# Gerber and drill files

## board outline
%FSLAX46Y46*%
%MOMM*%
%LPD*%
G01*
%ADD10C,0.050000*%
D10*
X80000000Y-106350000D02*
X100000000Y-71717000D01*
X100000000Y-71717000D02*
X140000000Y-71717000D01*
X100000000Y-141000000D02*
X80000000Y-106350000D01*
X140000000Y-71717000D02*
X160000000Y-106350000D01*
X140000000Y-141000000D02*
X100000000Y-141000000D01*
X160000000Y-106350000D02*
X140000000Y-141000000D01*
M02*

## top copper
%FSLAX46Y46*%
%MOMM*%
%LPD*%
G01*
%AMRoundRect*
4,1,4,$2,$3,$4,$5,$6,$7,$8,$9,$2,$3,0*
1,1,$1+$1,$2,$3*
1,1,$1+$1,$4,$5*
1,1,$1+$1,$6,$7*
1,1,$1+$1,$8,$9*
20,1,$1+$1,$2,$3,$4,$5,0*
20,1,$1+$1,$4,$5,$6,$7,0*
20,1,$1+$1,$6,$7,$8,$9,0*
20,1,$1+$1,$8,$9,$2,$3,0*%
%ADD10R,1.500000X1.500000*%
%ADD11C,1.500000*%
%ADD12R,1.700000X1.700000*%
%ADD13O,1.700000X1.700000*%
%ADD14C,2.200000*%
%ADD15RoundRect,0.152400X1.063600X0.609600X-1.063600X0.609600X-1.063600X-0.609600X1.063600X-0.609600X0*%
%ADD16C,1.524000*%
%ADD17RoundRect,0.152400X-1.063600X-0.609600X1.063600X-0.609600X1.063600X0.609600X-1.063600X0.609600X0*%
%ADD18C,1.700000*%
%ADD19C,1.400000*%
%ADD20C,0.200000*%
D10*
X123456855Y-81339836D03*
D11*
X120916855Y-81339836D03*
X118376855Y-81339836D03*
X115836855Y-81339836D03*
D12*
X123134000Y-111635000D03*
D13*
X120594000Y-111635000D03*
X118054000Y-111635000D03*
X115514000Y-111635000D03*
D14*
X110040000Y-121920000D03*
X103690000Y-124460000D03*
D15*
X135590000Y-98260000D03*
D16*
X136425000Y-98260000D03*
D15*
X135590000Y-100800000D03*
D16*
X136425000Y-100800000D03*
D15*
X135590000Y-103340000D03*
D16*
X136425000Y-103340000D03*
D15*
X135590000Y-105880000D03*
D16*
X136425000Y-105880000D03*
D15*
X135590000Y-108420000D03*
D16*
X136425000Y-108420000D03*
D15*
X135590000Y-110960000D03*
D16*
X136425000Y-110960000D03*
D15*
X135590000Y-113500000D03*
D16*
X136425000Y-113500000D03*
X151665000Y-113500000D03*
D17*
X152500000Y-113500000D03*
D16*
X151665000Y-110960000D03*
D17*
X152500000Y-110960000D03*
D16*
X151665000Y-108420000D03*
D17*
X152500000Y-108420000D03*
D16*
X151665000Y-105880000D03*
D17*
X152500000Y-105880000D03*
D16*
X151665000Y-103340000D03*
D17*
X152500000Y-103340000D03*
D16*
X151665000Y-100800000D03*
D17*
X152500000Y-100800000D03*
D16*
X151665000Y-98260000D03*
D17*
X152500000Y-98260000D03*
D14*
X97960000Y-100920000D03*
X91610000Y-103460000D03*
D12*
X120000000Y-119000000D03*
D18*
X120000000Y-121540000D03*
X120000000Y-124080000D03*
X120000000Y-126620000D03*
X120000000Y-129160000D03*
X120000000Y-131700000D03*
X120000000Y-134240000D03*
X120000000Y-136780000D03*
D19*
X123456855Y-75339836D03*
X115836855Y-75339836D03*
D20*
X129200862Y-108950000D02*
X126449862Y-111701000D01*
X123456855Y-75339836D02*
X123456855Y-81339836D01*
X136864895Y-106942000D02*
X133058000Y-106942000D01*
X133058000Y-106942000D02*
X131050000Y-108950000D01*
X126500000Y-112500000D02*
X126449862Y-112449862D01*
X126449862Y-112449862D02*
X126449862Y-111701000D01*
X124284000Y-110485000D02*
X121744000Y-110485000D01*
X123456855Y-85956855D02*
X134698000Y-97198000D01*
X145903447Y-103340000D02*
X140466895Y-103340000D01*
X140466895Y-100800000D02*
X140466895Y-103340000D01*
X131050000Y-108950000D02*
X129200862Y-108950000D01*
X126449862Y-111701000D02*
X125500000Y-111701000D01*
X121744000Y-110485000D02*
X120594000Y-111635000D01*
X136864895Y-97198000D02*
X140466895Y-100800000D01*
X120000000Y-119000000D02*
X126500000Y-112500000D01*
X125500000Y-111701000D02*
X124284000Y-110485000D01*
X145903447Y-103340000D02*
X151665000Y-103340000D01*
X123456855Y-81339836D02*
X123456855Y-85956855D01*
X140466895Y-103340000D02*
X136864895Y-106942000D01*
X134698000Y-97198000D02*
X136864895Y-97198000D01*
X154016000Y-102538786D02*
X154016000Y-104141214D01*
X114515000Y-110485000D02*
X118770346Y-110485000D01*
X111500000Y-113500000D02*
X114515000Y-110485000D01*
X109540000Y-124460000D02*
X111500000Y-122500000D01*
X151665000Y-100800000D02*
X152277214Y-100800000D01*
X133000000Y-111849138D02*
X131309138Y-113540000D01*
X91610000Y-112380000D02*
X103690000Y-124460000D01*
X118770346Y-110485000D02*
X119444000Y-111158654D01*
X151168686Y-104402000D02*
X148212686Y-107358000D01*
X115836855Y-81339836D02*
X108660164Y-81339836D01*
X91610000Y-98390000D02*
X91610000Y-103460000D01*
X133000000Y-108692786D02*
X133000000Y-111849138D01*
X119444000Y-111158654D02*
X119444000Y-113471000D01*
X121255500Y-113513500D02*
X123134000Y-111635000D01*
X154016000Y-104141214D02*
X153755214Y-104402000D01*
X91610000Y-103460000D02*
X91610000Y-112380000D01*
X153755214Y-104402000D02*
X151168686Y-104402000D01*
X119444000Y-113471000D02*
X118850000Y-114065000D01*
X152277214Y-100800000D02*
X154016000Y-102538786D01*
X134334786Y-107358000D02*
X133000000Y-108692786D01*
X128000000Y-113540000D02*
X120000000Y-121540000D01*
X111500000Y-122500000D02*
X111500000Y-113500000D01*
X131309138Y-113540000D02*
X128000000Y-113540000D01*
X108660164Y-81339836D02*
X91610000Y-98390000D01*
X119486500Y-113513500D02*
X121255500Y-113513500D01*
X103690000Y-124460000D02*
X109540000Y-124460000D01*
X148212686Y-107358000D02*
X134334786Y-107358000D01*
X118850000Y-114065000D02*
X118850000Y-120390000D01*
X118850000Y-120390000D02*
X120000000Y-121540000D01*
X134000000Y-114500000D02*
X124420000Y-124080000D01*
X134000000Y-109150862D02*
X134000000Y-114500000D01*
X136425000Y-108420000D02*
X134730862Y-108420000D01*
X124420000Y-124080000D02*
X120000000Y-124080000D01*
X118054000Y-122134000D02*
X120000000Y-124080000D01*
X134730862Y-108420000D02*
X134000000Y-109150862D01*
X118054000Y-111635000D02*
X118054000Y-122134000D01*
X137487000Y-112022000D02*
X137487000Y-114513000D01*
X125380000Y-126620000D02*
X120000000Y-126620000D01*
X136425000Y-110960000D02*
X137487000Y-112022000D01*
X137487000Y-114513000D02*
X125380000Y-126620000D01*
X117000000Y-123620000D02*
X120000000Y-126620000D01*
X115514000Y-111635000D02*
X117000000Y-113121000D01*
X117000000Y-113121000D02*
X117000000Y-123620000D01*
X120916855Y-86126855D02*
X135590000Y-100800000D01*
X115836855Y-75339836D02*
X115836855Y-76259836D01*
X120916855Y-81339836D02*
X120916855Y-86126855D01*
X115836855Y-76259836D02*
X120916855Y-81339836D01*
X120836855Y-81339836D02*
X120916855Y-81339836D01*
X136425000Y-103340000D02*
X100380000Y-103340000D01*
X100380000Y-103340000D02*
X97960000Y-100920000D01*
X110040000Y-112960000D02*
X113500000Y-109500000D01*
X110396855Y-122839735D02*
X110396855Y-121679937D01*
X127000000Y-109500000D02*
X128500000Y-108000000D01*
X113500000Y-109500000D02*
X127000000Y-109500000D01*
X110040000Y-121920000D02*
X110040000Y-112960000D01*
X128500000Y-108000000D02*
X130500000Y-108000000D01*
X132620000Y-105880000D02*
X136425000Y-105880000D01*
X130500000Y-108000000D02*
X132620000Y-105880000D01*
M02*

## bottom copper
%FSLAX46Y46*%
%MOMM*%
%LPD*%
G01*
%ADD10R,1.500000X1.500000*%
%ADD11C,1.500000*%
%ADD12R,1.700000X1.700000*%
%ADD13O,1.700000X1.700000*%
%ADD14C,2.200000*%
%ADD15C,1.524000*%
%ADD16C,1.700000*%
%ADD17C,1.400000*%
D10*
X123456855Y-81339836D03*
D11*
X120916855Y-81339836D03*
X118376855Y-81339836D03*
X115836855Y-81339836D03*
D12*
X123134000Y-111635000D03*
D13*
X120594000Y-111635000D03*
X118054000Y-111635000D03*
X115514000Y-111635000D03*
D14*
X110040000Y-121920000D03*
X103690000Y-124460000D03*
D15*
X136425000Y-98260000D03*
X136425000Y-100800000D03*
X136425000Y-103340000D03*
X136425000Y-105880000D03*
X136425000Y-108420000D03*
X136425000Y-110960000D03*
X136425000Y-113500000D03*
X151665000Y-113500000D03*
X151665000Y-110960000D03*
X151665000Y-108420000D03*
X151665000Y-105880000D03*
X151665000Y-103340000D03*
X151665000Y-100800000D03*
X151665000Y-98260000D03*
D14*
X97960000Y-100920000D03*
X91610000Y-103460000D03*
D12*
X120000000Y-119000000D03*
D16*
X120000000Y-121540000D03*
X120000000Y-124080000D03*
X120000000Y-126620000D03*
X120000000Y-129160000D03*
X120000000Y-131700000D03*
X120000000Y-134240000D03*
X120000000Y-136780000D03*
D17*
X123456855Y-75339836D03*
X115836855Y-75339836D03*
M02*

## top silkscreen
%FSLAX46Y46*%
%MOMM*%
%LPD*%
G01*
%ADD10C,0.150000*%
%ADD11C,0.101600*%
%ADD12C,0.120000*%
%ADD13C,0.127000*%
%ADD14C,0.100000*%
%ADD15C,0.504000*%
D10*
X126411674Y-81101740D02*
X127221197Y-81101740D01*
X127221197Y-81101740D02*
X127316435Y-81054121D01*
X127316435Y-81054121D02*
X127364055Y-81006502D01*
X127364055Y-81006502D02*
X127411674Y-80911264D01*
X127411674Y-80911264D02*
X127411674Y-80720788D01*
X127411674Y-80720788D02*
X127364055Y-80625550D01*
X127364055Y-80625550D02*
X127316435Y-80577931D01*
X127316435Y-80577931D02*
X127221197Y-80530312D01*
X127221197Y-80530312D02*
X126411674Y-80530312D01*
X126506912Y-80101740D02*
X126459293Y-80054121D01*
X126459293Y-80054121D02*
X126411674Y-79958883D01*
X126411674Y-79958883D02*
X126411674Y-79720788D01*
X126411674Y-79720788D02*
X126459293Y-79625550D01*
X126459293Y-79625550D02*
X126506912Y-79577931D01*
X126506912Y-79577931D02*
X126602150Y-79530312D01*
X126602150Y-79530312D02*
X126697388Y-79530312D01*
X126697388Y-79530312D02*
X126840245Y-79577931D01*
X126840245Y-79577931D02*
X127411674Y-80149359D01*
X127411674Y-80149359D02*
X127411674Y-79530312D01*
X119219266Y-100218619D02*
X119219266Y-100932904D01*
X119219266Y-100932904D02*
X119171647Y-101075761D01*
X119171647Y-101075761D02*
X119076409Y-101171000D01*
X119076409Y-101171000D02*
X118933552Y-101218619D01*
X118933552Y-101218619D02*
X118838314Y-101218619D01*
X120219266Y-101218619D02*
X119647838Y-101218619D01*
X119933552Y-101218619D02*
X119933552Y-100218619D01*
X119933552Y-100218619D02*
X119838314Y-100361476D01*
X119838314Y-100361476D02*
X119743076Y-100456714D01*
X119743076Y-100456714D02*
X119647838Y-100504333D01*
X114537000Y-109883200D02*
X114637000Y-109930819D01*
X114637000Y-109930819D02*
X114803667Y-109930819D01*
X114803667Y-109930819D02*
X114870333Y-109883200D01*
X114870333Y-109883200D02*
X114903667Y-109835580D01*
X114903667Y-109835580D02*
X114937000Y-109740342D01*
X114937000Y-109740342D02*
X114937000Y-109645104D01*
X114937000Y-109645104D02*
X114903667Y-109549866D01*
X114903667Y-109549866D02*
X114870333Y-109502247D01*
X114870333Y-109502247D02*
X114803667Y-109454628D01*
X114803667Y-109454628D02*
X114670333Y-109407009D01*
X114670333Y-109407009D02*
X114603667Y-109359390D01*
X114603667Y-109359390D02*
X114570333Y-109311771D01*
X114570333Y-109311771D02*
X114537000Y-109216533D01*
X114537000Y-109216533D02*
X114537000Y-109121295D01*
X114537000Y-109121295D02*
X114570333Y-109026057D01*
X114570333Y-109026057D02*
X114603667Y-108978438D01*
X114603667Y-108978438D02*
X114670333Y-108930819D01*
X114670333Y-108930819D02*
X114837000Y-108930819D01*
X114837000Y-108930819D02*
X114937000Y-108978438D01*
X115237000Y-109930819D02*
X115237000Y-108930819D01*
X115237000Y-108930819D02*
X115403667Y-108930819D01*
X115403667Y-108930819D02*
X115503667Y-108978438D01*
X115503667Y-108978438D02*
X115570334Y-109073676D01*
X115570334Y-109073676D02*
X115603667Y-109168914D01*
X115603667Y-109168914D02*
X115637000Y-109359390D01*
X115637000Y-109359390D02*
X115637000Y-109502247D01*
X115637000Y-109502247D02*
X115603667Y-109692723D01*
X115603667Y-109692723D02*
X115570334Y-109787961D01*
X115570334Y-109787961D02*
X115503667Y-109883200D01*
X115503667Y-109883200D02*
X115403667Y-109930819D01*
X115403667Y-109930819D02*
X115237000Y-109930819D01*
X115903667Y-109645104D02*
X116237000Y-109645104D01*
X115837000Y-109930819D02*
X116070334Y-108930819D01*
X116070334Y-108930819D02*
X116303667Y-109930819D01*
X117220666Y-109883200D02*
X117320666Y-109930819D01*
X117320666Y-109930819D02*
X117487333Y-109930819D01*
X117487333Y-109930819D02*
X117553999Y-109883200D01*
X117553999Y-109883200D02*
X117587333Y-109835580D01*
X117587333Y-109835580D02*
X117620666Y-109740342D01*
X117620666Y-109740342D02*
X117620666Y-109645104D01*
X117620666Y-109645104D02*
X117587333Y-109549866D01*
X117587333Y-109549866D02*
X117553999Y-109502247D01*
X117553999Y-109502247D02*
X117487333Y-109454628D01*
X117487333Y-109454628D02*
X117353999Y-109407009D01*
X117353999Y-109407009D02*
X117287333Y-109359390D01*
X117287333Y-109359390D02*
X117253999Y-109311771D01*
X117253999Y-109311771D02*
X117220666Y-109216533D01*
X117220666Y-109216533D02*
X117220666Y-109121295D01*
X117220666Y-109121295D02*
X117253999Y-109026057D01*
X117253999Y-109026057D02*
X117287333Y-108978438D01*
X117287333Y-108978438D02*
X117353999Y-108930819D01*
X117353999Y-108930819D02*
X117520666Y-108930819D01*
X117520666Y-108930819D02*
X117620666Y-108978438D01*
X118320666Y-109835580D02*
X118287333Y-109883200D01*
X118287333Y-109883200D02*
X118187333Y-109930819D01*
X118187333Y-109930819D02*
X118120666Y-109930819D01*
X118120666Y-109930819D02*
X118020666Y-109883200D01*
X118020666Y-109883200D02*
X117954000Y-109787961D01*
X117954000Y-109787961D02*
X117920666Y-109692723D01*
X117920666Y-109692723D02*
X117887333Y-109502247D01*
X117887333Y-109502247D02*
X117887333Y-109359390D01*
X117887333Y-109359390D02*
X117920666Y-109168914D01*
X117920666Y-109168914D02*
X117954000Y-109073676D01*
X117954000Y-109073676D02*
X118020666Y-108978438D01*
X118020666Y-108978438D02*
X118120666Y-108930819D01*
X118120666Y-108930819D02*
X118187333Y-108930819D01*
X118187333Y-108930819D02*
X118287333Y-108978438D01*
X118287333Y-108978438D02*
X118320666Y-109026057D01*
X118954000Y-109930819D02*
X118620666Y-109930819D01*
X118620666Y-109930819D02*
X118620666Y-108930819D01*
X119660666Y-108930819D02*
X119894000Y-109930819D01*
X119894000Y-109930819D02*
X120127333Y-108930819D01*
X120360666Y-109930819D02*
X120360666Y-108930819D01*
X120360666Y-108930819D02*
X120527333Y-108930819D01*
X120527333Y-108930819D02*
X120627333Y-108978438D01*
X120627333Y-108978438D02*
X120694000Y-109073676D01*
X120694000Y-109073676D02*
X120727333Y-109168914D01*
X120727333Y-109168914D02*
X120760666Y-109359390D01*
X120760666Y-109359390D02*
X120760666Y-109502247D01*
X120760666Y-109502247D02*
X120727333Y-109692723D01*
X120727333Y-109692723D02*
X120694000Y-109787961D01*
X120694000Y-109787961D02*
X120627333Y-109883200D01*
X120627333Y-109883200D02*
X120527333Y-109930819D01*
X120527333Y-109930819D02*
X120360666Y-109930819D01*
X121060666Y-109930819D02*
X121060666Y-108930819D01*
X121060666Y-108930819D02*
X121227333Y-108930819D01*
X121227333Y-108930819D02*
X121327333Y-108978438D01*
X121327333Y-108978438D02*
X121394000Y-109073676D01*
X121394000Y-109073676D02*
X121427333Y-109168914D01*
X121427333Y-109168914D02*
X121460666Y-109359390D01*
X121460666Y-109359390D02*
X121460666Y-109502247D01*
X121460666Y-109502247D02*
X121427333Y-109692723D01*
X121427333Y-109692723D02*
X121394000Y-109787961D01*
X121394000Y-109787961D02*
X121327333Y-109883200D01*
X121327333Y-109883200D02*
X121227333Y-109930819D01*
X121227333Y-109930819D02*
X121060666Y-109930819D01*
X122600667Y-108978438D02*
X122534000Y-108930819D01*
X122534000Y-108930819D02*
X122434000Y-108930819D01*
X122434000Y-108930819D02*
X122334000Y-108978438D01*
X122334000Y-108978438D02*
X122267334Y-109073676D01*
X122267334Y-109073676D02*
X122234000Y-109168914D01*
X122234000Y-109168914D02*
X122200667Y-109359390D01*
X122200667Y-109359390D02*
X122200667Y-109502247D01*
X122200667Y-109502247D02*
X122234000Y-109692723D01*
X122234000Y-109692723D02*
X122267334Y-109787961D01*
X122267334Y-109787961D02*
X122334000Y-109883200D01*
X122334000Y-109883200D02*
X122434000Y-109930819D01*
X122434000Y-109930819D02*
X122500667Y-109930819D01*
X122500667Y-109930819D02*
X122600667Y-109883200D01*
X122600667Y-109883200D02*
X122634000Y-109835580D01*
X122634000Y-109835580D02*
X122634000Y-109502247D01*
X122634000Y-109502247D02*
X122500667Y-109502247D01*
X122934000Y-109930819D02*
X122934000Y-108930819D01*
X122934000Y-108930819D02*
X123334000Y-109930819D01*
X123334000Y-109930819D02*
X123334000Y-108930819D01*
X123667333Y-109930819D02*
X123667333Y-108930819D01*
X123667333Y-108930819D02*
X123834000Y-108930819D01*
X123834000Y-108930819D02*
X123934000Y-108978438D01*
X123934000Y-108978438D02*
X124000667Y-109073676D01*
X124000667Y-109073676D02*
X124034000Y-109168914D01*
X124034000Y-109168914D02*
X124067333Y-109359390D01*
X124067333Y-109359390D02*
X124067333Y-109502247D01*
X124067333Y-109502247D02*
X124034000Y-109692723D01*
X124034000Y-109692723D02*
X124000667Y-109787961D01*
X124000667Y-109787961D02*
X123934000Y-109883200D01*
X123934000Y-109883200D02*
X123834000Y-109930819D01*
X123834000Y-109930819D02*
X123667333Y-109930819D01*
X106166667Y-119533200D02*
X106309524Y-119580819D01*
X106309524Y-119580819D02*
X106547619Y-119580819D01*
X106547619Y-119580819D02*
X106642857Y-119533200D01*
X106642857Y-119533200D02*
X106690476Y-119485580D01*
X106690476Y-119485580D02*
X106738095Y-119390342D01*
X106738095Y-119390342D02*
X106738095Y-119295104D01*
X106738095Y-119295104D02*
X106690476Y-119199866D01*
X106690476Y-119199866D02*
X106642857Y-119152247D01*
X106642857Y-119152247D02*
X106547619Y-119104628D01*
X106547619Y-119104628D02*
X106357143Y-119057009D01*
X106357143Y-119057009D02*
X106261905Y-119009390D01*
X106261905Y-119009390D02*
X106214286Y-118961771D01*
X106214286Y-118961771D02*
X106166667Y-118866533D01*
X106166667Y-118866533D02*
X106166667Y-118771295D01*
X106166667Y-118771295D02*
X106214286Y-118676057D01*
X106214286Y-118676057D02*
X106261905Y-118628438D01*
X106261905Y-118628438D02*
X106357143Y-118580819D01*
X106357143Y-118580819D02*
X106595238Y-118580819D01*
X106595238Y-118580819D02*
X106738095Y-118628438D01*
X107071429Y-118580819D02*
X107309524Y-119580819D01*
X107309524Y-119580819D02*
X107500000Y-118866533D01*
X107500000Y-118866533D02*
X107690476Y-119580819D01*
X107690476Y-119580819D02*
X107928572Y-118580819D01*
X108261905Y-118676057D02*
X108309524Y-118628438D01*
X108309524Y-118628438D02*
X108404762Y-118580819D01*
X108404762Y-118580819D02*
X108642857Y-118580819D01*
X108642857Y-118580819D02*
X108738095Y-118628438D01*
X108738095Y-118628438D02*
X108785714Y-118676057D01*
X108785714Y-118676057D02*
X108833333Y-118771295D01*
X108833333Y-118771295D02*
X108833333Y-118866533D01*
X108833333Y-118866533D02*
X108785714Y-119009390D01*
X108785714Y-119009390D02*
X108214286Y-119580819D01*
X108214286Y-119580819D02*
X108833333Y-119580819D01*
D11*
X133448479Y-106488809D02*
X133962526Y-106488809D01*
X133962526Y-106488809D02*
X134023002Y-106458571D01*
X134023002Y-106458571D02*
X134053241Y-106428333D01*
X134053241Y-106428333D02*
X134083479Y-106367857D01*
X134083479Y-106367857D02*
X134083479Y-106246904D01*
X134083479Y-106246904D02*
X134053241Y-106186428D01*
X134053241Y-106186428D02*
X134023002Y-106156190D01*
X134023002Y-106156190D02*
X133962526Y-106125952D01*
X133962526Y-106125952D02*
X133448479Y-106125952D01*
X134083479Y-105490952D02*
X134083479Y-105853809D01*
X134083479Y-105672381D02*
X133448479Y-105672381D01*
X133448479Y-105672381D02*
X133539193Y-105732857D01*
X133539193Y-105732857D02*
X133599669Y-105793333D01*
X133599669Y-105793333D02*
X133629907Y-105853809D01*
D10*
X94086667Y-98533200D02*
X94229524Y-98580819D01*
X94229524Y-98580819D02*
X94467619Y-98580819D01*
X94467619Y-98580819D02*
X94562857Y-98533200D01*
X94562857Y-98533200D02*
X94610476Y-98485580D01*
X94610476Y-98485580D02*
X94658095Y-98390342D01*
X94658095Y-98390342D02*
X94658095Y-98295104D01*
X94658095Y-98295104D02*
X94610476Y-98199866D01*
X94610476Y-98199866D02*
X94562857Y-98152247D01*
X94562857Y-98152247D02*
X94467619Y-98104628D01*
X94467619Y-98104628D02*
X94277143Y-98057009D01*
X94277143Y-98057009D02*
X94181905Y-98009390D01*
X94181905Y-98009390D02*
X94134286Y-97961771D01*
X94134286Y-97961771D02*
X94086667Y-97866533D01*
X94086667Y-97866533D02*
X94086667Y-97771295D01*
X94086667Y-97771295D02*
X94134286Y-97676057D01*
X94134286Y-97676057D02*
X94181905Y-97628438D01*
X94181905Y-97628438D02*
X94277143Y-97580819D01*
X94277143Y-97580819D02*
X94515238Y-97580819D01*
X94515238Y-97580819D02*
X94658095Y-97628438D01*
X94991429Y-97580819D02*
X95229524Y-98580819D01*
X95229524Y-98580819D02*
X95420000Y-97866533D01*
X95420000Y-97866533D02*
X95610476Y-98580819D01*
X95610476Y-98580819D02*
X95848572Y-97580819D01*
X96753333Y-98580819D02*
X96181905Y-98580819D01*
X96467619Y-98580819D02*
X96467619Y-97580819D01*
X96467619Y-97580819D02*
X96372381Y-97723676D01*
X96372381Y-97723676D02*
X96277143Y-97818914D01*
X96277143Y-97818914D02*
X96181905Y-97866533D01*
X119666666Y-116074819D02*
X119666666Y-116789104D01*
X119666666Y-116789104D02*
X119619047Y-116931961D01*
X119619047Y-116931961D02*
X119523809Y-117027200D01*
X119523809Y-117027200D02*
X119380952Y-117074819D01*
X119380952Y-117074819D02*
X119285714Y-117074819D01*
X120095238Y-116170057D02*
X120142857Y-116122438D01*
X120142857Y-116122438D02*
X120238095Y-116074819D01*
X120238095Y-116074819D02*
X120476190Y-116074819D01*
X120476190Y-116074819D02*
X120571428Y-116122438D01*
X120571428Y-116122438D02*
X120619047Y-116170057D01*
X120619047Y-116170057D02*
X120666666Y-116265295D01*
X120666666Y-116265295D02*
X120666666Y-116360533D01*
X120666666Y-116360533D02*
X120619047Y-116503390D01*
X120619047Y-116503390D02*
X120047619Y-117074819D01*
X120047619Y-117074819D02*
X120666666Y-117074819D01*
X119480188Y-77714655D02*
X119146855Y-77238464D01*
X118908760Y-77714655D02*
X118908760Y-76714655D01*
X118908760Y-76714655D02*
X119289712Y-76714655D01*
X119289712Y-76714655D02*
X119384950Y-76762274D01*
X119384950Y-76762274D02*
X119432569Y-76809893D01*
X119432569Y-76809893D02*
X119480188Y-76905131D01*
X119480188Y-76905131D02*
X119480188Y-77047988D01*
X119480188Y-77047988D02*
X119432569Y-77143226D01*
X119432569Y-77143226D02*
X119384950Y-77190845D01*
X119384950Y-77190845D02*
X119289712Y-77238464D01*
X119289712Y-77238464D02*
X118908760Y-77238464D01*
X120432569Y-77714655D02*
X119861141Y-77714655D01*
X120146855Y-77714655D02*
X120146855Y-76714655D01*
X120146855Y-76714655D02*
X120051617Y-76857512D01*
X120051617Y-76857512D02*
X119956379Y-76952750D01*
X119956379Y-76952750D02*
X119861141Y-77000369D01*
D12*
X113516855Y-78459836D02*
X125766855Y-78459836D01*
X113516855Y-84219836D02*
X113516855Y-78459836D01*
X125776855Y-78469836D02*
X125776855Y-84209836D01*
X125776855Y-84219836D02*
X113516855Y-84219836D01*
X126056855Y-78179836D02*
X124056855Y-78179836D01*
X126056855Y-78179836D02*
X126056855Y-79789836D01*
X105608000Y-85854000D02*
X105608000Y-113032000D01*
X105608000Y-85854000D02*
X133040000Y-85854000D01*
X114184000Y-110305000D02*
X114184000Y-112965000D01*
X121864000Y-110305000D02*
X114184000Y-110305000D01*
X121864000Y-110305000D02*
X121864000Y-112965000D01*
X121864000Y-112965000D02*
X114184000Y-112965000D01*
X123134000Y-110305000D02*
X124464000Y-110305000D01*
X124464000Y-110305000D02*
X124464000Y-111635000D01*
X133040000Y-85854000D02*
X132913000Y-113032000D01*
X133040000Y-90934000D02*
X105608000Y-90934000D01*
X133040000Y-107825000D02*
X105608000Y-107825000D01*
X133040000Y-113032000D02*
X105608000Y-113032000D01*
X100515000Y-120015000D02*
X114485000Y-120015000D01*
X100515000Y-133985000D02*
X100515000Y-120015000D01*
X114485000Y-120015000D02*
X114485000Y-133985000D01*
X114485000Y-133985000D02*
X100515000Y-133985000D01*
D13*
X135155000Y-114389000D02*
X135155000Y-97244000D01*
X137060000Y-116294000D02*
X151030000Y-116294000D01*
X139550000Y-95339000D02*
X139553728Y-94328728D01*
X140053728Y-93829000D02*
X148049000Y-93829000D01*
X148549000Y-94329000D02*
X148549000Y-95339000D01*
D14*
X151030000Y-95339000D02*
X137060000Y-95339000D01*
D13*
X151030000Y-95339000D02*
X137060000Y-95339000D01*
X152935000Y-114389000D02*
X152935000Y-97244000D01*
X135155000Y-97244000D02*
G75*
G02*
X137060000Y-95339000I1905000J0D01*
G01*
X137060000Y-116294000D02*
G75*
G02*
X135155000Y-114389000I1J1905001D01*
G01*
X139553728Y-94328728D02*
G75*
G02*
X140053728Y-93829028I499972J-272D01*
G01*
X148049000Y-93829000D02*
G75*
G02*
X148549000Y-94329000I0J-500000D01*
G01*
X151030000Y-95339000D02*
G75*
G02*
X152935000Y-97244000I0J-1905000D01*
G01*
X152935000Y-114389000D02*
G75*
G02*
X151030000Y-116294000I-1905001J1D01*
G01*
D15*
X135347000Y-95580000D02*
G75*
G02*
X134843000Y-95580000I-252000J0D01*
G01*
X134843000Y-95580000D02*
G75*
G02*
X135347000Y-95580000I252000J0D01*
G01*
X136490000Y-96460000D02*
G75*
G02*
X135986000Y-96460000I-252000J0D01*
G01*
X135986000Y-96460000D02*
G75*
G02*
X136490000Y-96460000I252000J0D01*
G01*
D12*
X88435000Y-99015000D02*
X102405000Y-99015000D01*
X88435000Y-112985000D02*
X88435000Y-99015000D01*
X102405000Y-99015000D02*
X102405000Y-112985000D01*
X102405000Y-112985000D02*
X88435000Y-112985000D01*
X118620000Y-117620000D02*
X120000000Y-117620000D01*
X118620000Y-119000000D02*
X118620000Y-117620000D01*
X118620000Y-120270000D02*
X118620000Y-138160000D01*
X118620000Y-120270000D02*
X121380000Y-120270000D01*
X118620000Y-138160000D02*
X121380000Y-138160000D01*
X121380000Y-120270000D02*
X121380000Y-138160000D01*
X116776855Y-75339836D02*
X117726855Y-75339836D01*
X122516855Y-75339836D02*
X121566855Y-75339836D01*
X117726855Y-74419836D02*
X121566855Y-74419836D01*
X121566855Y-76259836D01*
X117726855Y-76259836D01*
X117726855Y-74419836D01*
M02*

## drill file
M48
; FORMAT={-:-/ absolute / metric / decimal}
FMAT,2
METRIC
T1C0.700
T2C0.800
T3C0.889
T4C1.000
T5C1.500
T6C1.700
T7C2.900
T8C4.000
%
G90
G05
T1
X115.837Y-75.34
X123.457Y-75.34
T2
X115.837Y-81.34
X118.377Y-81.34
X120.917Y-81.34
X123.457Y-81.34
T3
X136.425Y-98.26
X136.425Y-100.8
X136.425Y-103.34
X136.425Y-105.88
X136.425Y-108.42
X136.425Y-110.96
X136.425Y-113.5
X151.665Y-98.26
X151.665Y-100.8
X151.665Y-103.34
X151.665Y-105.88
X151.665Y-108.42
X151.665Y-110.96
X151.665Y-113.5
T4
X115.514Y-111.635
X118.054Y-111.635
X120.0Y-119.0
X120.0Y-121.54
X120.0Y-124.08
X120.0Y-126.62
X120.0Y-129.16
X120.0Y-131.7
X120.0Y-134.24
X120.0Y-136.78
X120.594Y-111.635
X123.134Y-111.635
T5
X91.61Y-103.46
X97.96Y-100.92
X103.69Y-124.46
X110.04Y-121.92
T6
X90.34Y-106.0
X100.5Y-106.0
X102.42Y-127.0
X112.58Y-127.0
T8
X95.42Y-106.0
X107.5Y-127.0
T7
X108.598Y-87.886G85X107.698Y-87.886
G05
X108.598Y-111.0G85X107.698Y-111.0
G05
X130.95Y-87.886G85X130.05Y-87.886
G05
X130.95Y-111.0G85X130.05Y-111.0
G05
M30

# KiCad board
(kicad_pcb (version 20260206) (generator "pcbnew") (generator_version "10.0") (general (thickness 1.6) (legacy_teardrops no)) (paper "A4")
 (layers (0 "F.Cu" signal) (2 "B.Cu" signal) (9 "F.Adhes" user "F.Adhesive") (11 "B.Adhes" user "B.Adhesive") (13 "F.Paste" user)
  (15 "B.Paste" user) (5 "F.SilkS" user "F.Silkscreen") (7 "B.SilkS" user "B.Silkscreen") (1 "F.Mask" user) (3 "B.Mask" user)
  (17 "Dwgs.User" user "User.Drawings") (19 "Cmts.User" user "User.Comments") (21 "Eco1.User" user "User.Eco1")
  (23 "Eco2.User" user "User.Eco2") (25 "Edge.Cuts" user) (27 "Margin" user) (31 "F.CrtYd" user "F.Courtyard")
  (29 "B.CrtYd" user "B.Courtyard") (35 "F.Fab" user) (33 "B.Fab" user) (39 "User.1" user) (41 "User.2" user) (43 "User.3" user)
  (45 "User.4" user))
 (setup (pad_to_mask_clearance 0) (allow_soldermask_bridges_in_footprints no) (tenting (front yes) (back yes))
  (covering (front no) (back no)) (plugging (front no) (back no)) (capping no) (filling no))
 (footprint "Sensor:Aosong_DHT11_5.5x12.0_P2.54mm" (layer "F.Cu") (at 123.456855 81.339836 -90)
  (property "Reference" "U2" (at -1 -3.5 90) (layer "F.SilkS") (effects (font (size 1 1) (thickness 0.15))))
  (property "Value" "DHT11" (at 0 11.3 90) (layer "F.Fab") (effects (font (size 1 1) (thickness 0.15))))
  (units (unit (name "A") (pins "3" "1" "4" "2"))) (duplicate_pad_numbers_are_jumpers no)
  (fp_line (start -2.88 9.94) (end -2.88 -2.31) (stroke (width 0.12) (type solid)) (layer "F.SilkS"))
  (fp_line (start 2.88 9.94) (end -2.88 9.94) (stroke (width 0.12) (type solid)) (layer "F.SilkS"))
  (fp_line (start -2.87 -2.32) (end 2.87 -2.32) (stroke (width 0.12) (type solid)) (layer "F.SilkS"))
  (fp_line (start 2.88 -2.32) (end 2.88 9.94) (stroke (width 0.12) (type solid)) (layer "F.SilkS"))
  (fp_line (start -3.16 -2.6) (end -3.16 -0.6) (stroke (width 0.12) (type solid)) (layer "F.SilkS"))
  (fp_line (start -3.16 -2.6) (end -1.55 -2.6) (stroke (width 0.12) (type solid)) (layer "F.SilkS"))
  (pad "1" thru_hole rect (at 0 0 270) (size 1.5 1.5) (drill 0.8) (layers "*.Cu" "*.Mask") (remove_unused_layers no) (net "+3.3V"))
  (pad "2" thru_hole circle (at 0 2.54 270) (size 1.5 1.5) (drill 0.8) (layers "*.Cu" "*.Mask") (remove_unused_layers no)
   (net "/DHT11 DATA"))
  (pad "3" thru_hole circle (at 0 5.08 270) (size 1.5 1.5) (drill 0.8) (layers "*.Cu" "*.Mask") (remove_unused_layers no)
   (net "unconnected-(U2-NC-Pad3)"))
  (pad "4" thru_hole circle (at 0 7.62 270) (size 1.5 1.5) (drill 0.8) (layers "*.Cu" "*.Mask") (remove_unused_layers no) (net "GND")))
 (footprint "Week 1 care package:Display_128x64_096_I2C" (layer "F.Cu") (at 119.324 111.635 180)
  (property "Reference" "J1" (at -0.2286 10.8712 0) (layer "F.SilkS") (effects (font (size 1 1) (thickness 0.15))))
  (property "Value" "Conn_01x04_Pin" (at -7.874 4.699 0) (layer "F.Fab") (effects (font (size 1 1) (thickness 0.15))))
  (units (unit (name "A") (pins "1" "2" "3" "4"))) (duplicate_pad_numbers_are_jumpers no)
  (fp_line (start 13.716 25.781) (end 13.716 -1.397) (stroke (width 0.12) (type solid)) (layer "F.SilkS"))
  (fp_line (start 13.716 25.781) (end -13.716 25.781) (stroke (width 0.12) (type solid)) (layer "F.SilkS"))
  (fp_line (start 5.14 1.33) (end 5.14 -1.33) (stroke (width 0.12) (type solid)) (layer "F.SilkS"))
  (fp_line (start -2.54 1.33) (end 5.14 1.33) (stroke (width 0.12) (type solid)) (layer "F.SilkS"))
  (fp_line (start -2.54 1.33) (end -2.54 -1.33) (stroke (width 0.12) (type solid)) (layer "F.SilkS"))
  (fp_line (start -2.54 -1.33) (end 5.14 -1.33) (stroke (width 0.12) (type solid)) (layer "F.SilkS"))
  (fp_line (start -3.81 1.33) (end -5.14 1.33) (stroke (width 0.12) (type solid)) (layer "F.SilkS"))
  (fp_line (start -5.14 1.33) (end -5.14 0) (stroke (width 0.12) (type solid)) (layer "F.SilkS"))
  (fp_line (start -13.716 25.781) (end -13.589 -1.397) (stroke (width 0.12) (type solid)) (layer "F.SilkS"))
  (fp_line (start -13.716 20.701) (end 13.716 20.701) (stroke (width 0.12) (type solid)) (layer "F.SilkS"))
  (fp_line (start -13.716 3.81) (end 13.716 3.81) (stroke (width 0.12) (type solid)) (layer "F.SilkS"))
  (fp_line (start -13.716 -1.397) (end 13.716 -1.397) (stroke (width 0.12) (type solid)) (layer "F.SilkS"))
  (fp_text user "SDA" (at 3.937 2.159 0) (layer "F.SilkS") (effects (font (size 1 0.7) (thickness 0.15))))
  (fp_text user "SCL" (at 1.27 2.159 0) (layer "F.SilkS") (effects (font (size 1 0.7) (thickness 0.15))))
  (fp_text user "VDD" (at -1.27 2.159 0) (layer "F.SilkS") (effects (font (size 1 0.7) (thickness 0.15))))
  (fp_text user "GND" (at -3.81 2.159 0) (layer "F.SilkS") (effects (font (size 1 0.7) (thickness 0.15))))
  (pad "" np_thru_hole oval (at -11.176 0.635 180) (size 3.8 2.9) (drill oval 3.8 2.9) (layers "*.Cu" "*.Mask"))
  (pad "" np_thru_hole oval (at -11.176 23.749 180) (size 3.8 2.9) (drill oval 3.8 2.9) (layers "*.Cu" "*.Mask"))
  (pad "" np_thru_hole oval (at 11.176 0.635 180) (size 3.8 2.9) (drill oval 3.8 2.9) (layers "*.Cu" "*.Mask"))
  (pad "" np_thru_hole oval (at 11.176 23.749 180) (size 3.8 2.9) (drill oval 3.8 2.9) (layers "*.Cu" "*.Mask"))
  (pad "1" thru_hole rect (at -3.81 0 270) (size 1.7 1.7) (drill 1) (layers "*.Cu" "*.Mask") (remove_unused_layers no) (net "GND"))
  (pad "2" thru_hole oval (at -1.27 0 270) (size 1.7 1.7) (drill 1) (layers "*.Cu" "*.Mask") (remove_unused_layers no) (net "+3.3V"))
  (pad "3" thru_hole oval (at 1.27 0 270) (size 1.7 1.7) (drill 1) (layers "*.Cu" "*.Mask") (remove_unused_layers no) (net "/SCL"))
  (pad "4" thru_hole oval (at 3.81 0 270) (size 1.7 1.7) (drill 1) (layers "*.Cu" "*.Mask") (remove_unused_layers no) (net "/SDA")))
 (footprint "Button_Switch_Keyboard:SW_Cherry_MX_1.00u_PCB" (layer "F.Cu") (at 110.04 121.92)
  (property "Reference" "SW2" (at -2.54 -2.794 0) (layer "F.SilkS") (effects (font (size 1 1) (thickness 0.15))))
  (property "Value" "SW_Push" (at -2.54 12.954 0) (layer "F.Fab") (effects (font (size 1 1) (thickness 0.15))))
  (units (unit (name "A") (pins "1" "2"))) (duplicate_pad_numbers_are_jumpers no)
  (fp_line (start -9.525 -1.905) (end 4.445 -1.905) (stroke (width 0.12) (type solid)) (layer "F.SilkS"))
  (fp_line (start -9.525 12.065) (end -9.525 -1.905) (stroke (width 0.12) (type solid)) (layer "F.SilkS"))
  (fp_line (start 4.445 -1.905) (end 4.445 12.065) (stroke (width 0.12) (type solid)) (layer "F.SilkS"))
  (fp_line (start 4.445 12.065) (end -9.525 12.065) (stroke (width 0.12) (type solid)) (layer "F.SilkS"))
  (pad "" np_thru_hole circle (at -7.62 5.08) (size 1.7 1.7) (drill 1.7) (layers "*.Cu" "*.Mask"))
  (pad "" np_thru_hole circle (at -2.54 5.08) (size 4 4) (drill 4) (layers "*.Cu" "*.Mask"))
  (pad "" np_thru_hole circle (at 2.54 5.08) (size 1.7 1.7) (drill 1.7) (layers "*.Cu" "*.Mask"))
  (pad "1" thru_hole circle (at 0 0) (size 2.2 2.2) (drill 1.5) (layers "*.Cu" "*.Mask") (remove_unused_layers no) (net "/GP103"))
  (pad "2" thru_hole circle (at -6.35 2.54) (size 2.2 2.2) (drill 1.5) (layers "*.Cu" "*.Mask") (remove_unused_layers no) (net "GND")))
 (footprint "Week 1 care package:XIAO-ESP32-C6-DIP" (layer "F.Cu") (at 144.045 105.88 90)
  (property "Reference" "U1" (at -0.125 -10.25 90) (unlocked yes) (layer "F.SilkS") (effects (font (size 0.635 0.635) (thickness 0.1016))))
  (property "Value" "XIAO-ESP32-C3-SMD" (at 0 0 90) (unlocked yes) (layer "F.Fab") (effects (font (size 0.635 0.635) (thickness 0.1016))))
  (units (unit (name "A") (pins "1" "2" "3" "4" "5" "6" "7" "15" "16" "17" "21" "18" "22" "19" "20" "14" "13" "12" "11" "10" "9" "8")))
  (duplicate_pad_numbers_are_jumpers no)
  (fp_line (start -8.509 -8.89) (end 8.636 -8.89) (stroke (width 0.127) (type solid)) (layer "F.SilkS"))
  (fp_line (start -10.414 -6.985) (end -10.414 6.985) (stroke (width 0.127) (type solid)) (layer "F.SilkS"))
  (fp_line (start 10.541 -4.495) (end 11.551272 -4.491272) (stroke (width 0.127) (type solid)) (layer "F.SilkS"))
  (fp_line (start 12.051 -3.991272) (end 12.051 4.004) (stroke (width 0.127) (type solid)) (layer "F.SilkS"))
  (fp_line (start 11.551 4.504) (end 10.541 4.504) (stroke (width 0.127) (type solid)) (layer "F.SilkS"))
  (fp_line (start 10.541 6.985) (end 10.541 -6.985) (stroke (width 0.1) (type solid)) (layer "F.SilkS"))
  (fp_line (start 10.541 6.985) (end 10.541 -6.985) (stroke (width 0.127) (type solid)) (layer "F.SilkS"))
  (fp_line (start -8.509 8.89) (end 8.636 8.89) (stroke (width 0.127) (type solid)) (layer "F.SilkS"))
  (fp_arc (start 8.636 -8.89) (mid 9.983038 -8.332038) (end 10.541 -6.985) (stroke (width 0.127) (type solid)) (layer "F.SilkS"))
  (fp_arc (start -10.414 -6.985) (mid -9.856038 -8.332038) (end -8.509 -8.89) (stroke (width 0.127) (type solid)) (layer "F.SilkS"))
  (fp_arc (start 11.551272 -4.491272) (mid 11.904644 -4.344724) (end 12.051 -3.991272) (stroke (width 0.127) (type default))
   (layer "F.SilkS"))
  (fp_arc (start 12.051 4.004) (mid 11.904553 4.357553) (end 11.551 4.504) (stroke (width 0.127) (type default)) (layer "F.SilkS"))
  (fp_arc (start 10.541 6.985) (mid 9.983038 8.332038) (end 8.636 8.89) (stroke (width 0.127) (type solid)) (layer "F.SilkS"))
  (fp_arc (start -8.509 8.89) (mid -9.856038 8.332038) (end -10.414 6.985) (stroke (width 0.127) (type solid)) (layer "F.SilkS"))
  (fp_circle (center 10.3 -8.95) (end 10.554 -8.95) (stroke (width 0.5) (type solid)) (fill yes) (layer "F.SilkS"))
  (fp_circle (center 9.42 -7.807) (end 9.674 -7.807) (stroke (width 0.5) (type solid)) (fill yes) (layer "F.SilkS"))
  (pad "1" smd roundrect (at 7.62 -8.455 180) (size 2.432 1.524) (layers "F.Cu" "F.Mask") (roundrect_rratio 0.1)
   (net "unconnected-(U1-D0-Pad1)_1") (thermal_bridge_angle 45))
  (pad "1" thru_hole circle (at 7.62 -7.62 180) (size 1.524 1.524) (drill 0.889) (layers "*.Cu" "*.Mask") (remove_unused_layers no)
   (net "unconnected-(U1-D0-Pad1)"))
  (pad "2" smd roundrect (at 5.08 -8.455 180) (size 2.432 1.524) (layers "F.Cu" "F.Mask") (roundrect_rratio 0.1) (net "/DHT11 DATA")
   (thermal_bridge_angle 45))
  (pad "2" thru_hole circle (at 5.08 -7.62 180) (size 1.524 1.524) (drill 0.889) (layers "*.Cu" "*.Mask") (remove_unused_layers no)
   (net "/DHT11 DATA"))
  (pad "3" smd roundrect (at 2.54 -8.455 180) (size 2.432 1.524) (layers "F.Cu" "F.Mask") (roundrect_rratio 0.1) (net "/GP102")
   (thermal_bridge_angle 45))
  (pad "3" thru_hole circle (at 2.54 -7.62 180) (size 1.524 1.524) (drill 0.889) (layers "*.Cu" "*.Mask") (remove_unused_layers no)
   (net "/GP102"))
  (pad "4" smd roundrect (at 0 -8.455 180) (size 2.432 1.524) (layers "F.Cu" "F.Mask") (roundrect_rratio 0.1) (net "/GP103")
   (thermal_bridge_angle 45))
  (pad "4" thru_hole circle (at 0 -7.62 180) (size 1.524 1.524) (drill 0.889) (layers "*.Cu" "*.Mask") (remove_unused_layers no)
   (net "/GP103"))
  (pad "5" smd roundrect (at -2.54 -8.455 180) (size 2.432 1.524) (layers "F.Cu" "F.Mask") (roundrect_rratio 0.1) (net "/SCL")
   (thermal_bridge_angle 45))
  (pad "5" thru_hole circle (at -2.54 -7.62 180) (size 1.524 1.524) (drill 0.889) (layers "*.Cu" "*.Mask") (remove_unused_layers no)
   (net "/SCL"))
  (pad "6" smd roundrect (at -5.08 -8.455 180) (size 2.432 1.524) (layers "F.Cu" "F.Mask") (roundrect_rratio 0.1) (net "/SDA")
   (thermal_bridge_angle 45))
  (pad "6" thru_hole circle (at -5.08 -7.62 180) (size 1.524 1.524) (drill 0.889) (layers "*.Cu" "*.Mask") (remove_unused_layers no)
   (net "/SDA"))
  (pad "7" smd roundrect (at -7.62 -8.455 180) (size 2.432 1.524) (layers "F.Cu" "F.Mask") (roundrect_rratio 0.1)
   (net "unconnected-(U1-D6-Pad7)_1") (thermal_bridge_angle 45))
  (pad "7" thru_hole circle (at -7.62 -7.62 180) (size 1.524 1.524) (drill 0.889) (layers "*.Cu" "*.Mask") (remove_unused_layers no)
   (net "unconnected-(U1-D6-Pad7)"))
  (pad "8" thru_hole circle (at -7.62 7.62) (size 1.524 1.524) (drill 0.889) (layers "*.Cu" "*.Mask") (remove_unused_layers no)
   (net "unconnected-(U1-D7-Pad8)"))
  (pad "8" smd roundrect (at -7.62 8.455) (size 2.432 1.524) (layers "F.Cu" "F.Mask") (roundrect_rratio 0.1)
   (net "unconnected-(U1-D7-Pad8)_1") (thermal_bridge_angle 45))
  (pad "9" thru_hole circle (at -5.08 7.62) (size 1.524 1.524) (drill 0.889) (layers "*.Cu" "*.Mask") (remove_unused_layers no)
   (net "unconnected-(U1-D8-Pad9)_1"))
  (pad "9" smd roundrect (at -5.08 8.455) (size 2.432 1.524) (layers "F.Cu" "F.Mask") (roundrect_rratio 0.1)
   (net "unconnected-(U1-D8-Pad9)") (thermal_bridge_angle 45))
  (pad "10" thru_hole circle (at -2.54 7.62) (size 1.524 1.524) (drill 0.889) (layers "*.Cu" "*.Mask") (remove_unused_layers no)
   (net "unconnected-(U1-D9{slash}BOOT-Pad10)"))
  (pad "10" smd roundrect (at -2.54 8.455) (size 2.432 1.524) (layers "F.Cu" "F.Mask") (roundrect_rratio 0.1)
   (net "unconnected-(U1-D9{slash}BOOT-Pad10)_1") (thermal_bridge_angle 45))
  (pad "11" thru_hole circle (at 0 7.62) (size 1.524 1.524) (drill 0.889) (layers "*.Cu" "*.Mask") (remove_unused_layers no)
   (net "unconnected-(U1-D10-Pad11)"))
  (pad "11" smd roundrect (at 0 8.455) (size 2.432 1.524) (layers "F.Cu" "F.Mask") (roundrect_rratio 0.1)
   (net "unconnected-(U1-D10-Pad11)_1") (thermal_bridge_angle 45))
  (pad "12" thru_hole circle (at 2.54 7.62) (size 1.524 1.524) (drill 0.889) (layers "*.Cu" "*.Mask") (remove_unused_layers no)
   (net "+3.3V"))
  (pad "12" smd roundrect (at 2.54 8.455) (size 2.432 1.524) (layers "F.Cu" "F.Mask") (roundrect_rratio 0.1) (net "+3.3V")
   (thermal_bridge_angle 45))
  (pad "13" thru_hole circle (at 5.08 7.62) (size 1.524 1.524) (drill 0.889) (layers "*.Cu" "*.Mask") (remove_unused_layers no) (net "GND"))
  (pad "13" smd roundrect (at 5.08 8.455) (size 2.432 1.524) (layers "F.Cu" "F.Mask") (roundrect_rratio 0.1) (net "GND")
   (thermal_bridge_angle 45))
  (pad "14" thru_hole circle (at 7.62 7.62) (size 1.524 1.524) (drill 0.889) (layers "*.Cu" "*.Mask") (remove_unused_layers no) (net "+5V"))
  (pad "14" smd roundrect (at 7.62 8.455) (size 2.432 1.524) (layers "F.Cu" "F.Mask") (roundrect_rratio 0.1) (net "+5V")
   (thermal_bridge_angle 45)))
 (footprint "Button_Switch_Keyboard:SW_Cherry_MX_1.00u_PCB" (layer "F.Cu") (at 97.96 100.92)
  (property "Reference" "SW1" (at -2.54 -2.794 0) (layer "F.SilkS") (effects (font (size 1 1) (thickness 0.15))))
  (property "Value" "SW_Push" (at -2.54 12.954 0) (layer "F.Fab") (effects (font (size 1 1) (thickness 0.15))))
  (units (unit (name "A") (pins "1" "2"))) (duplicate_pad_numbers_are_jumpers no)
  (fp_line (start -9.525 -1.905) (end 4.445 -1.905) (stroke (width 0.12) (type solid)) (layer "F.SilkS"))
  (fp_line (start -9.525 12.065) (end -9.525 -1.905) (stroke (width 0.12) (type solid)) (layer "F.SilkS"))
  (fp_line (start 4.445 -1.905) (end 4.445 12.065) (stroke (width 0.12) (type solid)) (layer "F.SilkS"))
  (fp_line (start 4.445 12.065) (end -9.525 12.065) (stroke (width 0.12) (type solid)) (layer "F.SilkS"))
  (pad "" np_thru_hole circle (at -7.62 5.08) (size 1.7 1.7) (drill 1.7) (layers "*.Cu" "*.Mask"))
  (pad "" np_thru_hole circle (at -2.54 5.08) (size 4 4) (drill 4) (layers "*.Cu" "*.Mask"))
  (pad "" np_thru_hole circle (at 2.54 5.08) (size 1.7 1.7) (drill 1.7) (layers "*.Cu" "*.Mask"))
  (pad "1" thru_hole circle (at 0 0) (size 2.2 2.2) (drill 1.5) (layers "*.Cu" "*.Mask") (remove_unused_layers no) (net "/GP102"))
  (pad "2" thru_hole circle (at -6.35 2.54) (size 2.2 2.2) (drill 1.5) (layers "*.Cu" "*.Mask") (remove_unused_layers no) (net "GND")))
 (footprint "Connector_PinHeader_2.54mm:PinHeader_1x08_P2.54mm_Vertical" (layer "F.Cu") (at 120 119)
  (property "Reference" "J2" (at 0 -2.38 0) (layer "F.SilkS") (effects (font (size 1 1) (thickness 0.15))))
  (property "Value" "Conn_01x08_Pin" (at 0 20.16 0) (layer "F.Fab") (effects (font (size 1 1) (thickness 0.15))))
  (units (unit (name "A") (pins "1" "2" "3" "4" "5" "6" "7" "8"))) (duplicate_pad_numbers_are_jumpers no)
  (fp_line (start -1.38 -1.38) (end 0 -1.38) (stroke (width 0.12) (type solid)) (layer "F.SilkS"))
  (fp_line (start -1.38 0) (end -1.38 -1.38) (stroke (width 0.12) (type solid)) (layer "F.SilkS"))
  (fp_line (start -1.38 1.27) (end -1.38 19.16) (stroke (width 0.12) (type solid)) (layer "F.SilkS"))
  (fp_line (start -1.38 1.27) (end 1.38 1.27) (stroke (width 0.12) (type solid)) (layer "F.SilkS"))
  (fp_line (start -1.38 19.16) (end 1.38 19.16) (stroke (width 0.12) (type solid)) (layer "F.SilkS"))
  (fp_line (start 1.38 1.27) (end 1.38 19.16) (stroke (width 0.12) (type solid)) (layer "F.SilkS"))
  (pad "1" thru_hole rect (at 0 0) (size 1.7 1.7) (drill 1) (layers "*.Cu" "*.Mask") (remove_unused_layers no) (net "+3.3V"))
  (pad "2" thru_hole circle (at 0 2.54) (size 1.7 1.7) (drill 1) (layers "*.Cu" "*.Mask") (remove_unused_layers no) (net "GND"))
  (pad "3" thru_hole circle (at 0 5.08) (size 1.7 1.7) (drill 1) (layers "*.Cu" "*.Mask") (remove_unused_layers no) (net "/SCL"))
  (pad "4" thru_hole circle (at 0 7.62) (size 1.7 1.7) (drill 1) (layers "*.Cu" "*.Mask") (remove_unused_layers no) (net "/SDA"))
  (pad "5" thru_hole circle (at 0 10.16) (size 1.7 1.7) (drill 1) (layers "*.Cu" "*.Mask") (remove_unused_layers no)
   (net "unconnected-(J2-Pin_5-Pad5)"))
  (pad "6" thru_hole circle (at 0 12.7) (size 1.7 1.7) (drill 1) (layers "*.Cu" "*.Mask") (remove_unused_layers no)
   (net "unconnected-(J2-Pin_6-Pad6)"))
  (pad "7" thru_hole circle (at 0 15.24) (size 1.7 1.7) (drill 1) (layers "*.Cu" "*.Mask") (remove_unused_layers no)
   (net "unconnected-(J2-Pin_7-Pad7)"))
  (pad "8" thru_hole circle (at 0 17.78) (size 1.7 1.7) (drill 1) (layers "*.Cu" "*.Mask") (remove_unused_layers no)
   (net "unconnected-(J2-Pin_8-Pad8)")))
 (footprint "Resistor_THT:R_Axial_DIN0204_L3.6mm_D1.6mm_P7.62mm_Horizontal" (layer "F.Cu") (at 123.456855 75.339836 180)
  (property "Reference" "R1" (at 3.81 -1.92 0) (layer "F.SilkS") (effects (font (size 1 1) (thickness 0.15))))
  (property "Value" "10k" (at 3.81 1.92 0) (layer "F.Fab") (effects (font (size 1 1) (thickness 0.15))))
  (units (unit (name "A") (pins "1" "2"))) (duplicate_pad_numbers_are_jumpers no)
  (fp_line (start 6.68 0) (end 5.73 0) (stroke (width 0.12) (type solid)) (layer "F.SilkS"))
  (fp_line (start 0.94 0) (end 1.89 0) (stroke (width 0.12) (type solid)) (layer "F.SilkS"))
  (fp_rect (start 1.89 -0.92) (end 5.73 0.92) (stroke (width 0.12) (type solid)) (fill no) (layer "F.SilkS"))
  (pad "1" thru_hole circle (at 0 0 180) (size 1.4 1.4) (drill 0.7) (layers "*.Cu" "*.Mask") (remove_unused_layers no) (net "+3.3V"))
  (pad "2" thru_hole circle (at 7.62 0 180) (size 1.4 1.4) (drill 0.7) (layers "*.Cu" "*.Mask") (remove_unused_layers no)
   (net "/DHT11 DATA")))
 (gr_line (start 80 106.35) (end 100 71.717) (stroke (width 0.05) (type default)) (layer "Edge.Cuts"))
 (gr_line (start 100 71.717) (end 140 71.717) (stroke (width 0.05) (type default)) (layer "Edge.Cuts"))
 (gr_line (start 100 141) (end 80 106.35) (stroke (width 0.05) (type default)) (layer "Edge.Cuts"))
 (gr_line (start 140 71.717) (end 160 106.35) (stroke (width 0.05) (type default)) (layer "Edge.Cuts"))
 (gr_line (start 140 141) (end 100 141) (stroke (width 0.05) (type default)) (layer "Edge.Cuts"))
 (gr_line (start 160 106.35) (end 140 141) (stroke (width 0.05) (type default)) (layer "Edge.Cuts"))
 (segment (start 129.200862 108.95) (end 126.449862 111.701) (width 0.2) (layer "F.Cu") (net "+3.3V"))
 (segment (start 123.456855 75.339836) (end 123.456855 81.339836) (width 0.2) (layer "F.Cu") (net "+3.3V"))
 (segment (start 136.864895 106.942) (end 133.058 106.942) (width 0.2) (layer "F.Cu") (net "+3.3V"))
 (segment (start 133.058 106.942) (end 131.05 108.95) (width 0.2) (layer "F.Cu") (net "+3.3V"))
 (segment (start 126.5 112.5) (end 126.449862 112.449862) (width 0.2) (layer "F.Cu") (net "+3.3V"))
 (segment (start 126.449862 112.449862) (end 126.449862 111.701) (width 0.2) (layer "F.Cu") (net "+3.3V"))
 (segment (start 124.284 110.485) (end 121.744 110.485) (width 0.2) (layer "F.Cu") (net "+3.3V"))
 (segment (start 123.456855 85.956855) (end 134.698 97.198) (width 0.2) (layer "F.Cu") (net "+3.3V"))
 (segment (start 145.903447 103.34) (end 140.466895 103.34) (width 0.2) (layer "F.Cu") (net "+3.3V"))
 (segment (start 140.466895 100.8) (end 140.466895 103.34) (width 0.2) (layer "F.Cu") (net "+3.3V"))
 (segment (start 131.05 108.95) (end 129.200862 108.95) (width 0.2) (layer "F.Cu") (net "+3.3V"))
 (segment (start 126.449862 111.701) (end 125.5 111.701) (width 0.2) (layer "F.Cu") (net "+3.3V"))
 (segment (start 121.744 110.485) (end 120.594 111.635) (width 0.2) (layer "F.Cu") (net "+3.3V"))
 (segment (start 136.864895 97.198) (end 140.466895 100.8) (width 0.2) (layer "F.Cu") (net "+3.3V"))
 (segment (start 120 119) (end 126.5 112.5) (width 0.2) (layer "F.Cu") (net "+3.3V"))
 (segment (start 125.5 111.701) (end 124.284 110.485) (width 0.2) (layer "F.Cu") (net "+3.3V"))
 (segment (start 145.903447 103.34) (end 151.665 103.34) (width 0.2) (layer "F.Cu") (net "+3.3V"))
 (segment (start 123.456855 81.339836) (end 123.456855 85.956855) (width 0.2) (layer "F.Cu") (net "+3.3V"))
 (segment (start 140.466895 103.34) (end 136.864895 106.942) (width 0.2) (layer "F.Cu") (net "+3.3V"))
 (segment (start 134.698 97.198) (end 136.864895 97.198) (width 0.2) (layer "F.Cu") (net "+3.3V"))
 (segment (start 154.016 102.538786) (end 154.016 104.141214) (width 0.2) (layer "F.Cu") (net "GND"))
 (segment (start 114.515 110.485) (end 118.770346 110.485) (width 0.2) (layer "F.Cu") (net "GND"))
 (segment (start 111.5 113.5) (end 114.515 110.485) (width 0.2) (layer "F.Cu") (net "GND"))
 (segment (start 109.54 124.46) (end 111.5 122.5) (width 0.2) (layer "F.Cu") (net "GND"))
 (segment (start 151.665 100.8) (end 152.277214 100.8) (width 0.2) (layer "F.Cu") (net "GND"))
 (segment (start 133 111.849138) (end 131.309138 113.54) (width 0.2) (layer "F.Cu") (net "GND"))
 (segment (start 91.61 112.38) (end 103.69 124.46) (width 0.2) (layer "F.Cu") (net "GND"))
 (segment (start 118.770346 110.485) (end 119.444 111.158654) (width 0.2) (layer "F.Cu") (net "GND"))
 (segment (start 151.168686 104.402) (end 148.212686 107.358) (width 0.2) (layer "F.Cu") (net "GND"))
 (segment (start 115.836855 81.339836) (end 108.660164 81.339836) (width 0.2) (layer "F.Cu") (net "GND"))
 (segment (start 91.61 98.39) (end 91.61 103.46) (width 0.2) (layer "F.Cu") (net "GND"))
 (segment (start 133 108.692786) (end 133 111.849138) (width 0.2) (layer "F.Cu") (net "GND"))
 (segment (start 119.444 111.158654) (end 119.444 113.471) (width 0.2) (layer "F.Cu") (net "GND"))
 (segment (start 121.2555 113.5135) (end 123.134 111.635) (width 0.2) (layer "F.Cu") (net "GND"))
 (segment (start 154.016 104.141214) (end 153.755214 104.402) (width 0.2) (layer "F.Cu") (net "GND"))
 (segment (start 91.61 103.46) (end 91.61 112.38) (width 0.2) (layer "F.Cu") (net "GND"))
 (segment (start 153.755214 104.402) (end 151.168686 104.402) (width 0.2) (layer "F.Cu") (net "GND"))
 (segment (start 119.444 113.471) (end 118.85 114.065) (width 0.2) (layer "F.Cu") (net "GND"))
 (segment (start 152.277214 100.8) (end 154.016 102.538786) (width 0.2) (layer "F.Cu") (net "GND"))
 (segment (start 134.334786 107.358) (end 133 108.692786) (width 0.2) (layer "F.Cu") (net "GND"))
 (segment (start 128 113.54) (end 120 121.54) (width 0.2) (layer "F.Cu") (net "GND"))
 (segment (start 111.5 122.5) (end 111.5 113.5) (width 0.2) (layer "F.Cu") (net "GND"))
 (segment (start 131.309138 113.54) (end 128 113.54) (width 0.2) (layer "F.Cu") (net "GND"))
 (segment (start 108.660164 81.339836) (end 91.61 98.39) (width 0.2) (layer "F.Cu") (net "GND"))
 (segment (start 119.4865 113.5135) (end 121.2555 113.5135) (width 0.2) (layer "F.Cu") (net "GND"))
 (segment (start 103.69 124.46) (end 109.54 124.46) (width 0.2) (layer "F.Cu") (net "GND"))
 (segment (start 148.212686 107.358) (end 134.334786 107.358) (width 0.2) (layer "F.Cu") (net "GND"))
 (segment (start 118.85 114.065) (end 118.85 120.39) (width 0.2) (layer "F.Cu") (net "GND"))
 (segment (start 118.85 120.39) (end 120 121.54) (width 0.2) (layer "F.Cu") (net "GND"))
 (segment (start 134 114.5) (end 124.42 124.08) (width 0.2) (layer "F.Cu") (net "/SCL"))
 (segment (start 134 109.150862) (end 134 114.5) (width 0.2) (layer "F.Cu") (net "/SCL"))
 (segment (start 136.425 108.42) (end 134.730862 108.42) (width 0.2) (layer "F.Cu") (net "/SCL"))
 (segment (start 124.42 124.08) (end 120 124.08) (width 0.2) (layer "F.Cu") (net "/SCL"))
 (segment (start 118.054 122.134) (end 120 124.08) (width 0.2) (layer "F.Cu") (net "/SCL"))
 (segment (start 134.730862 108.42) (end 134 109.150862) (width 0.2) (layer "F.Cu") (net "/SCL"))
 (segment (start 118.054 111.635) (end 118.054 122.134) (width 0.2) (layer "F.Cu") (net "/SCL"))
 (segment (start 137.487 112.022) (end 137.487 114.513) (width 0.2) (layer "F.Cu") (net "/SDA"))
 (segment (start 125.38 126.62) (end 120 126.62) (width 0.2) (layer "F.Cu") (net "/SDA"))
 (segment (start 136.425 110.96) (end 137.487 112.022) (width 0.2) (layer "F.Cu") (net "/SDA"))
 (segment (start 137.487 114.513) (end 125.38 126.62) (width 0.2) (layer "F.Cu") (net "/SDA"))
 (segment (start 117 123.62) (end 120 126.62) (width 0.2) (layer "F.Cu") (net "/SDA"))
 (segment (start 115.514 111.635) (end 117 113.121) (width 0.2) (layer "F.Cu") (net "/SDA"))
 (segment (start 117 113.121) (end 117 123.62) (width 0.2) (layer "F.Cu") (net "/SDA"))
 (segment (start 120.916855 86.126855) (end 135.59 100.8) (width 0.2) (layer "F.Cu") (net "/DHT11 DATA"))
 (segment (start 115.836855 75.339836) (end 115.836855 76.259836) (width 0.2) (layer "F.Cu") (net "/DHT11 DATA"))
 (segment (start 120.916855 81.339836) (end 120.916855 86.126855) (width 0.2) (layer "F.Cu") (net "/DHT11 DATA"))
 (segment (start 115.836855 76.259836) (end 120.916855 81.339836) (width 0.2) (layer "F.Cu") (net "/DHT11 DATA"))
 (segment (start 120.836855 81.339836) (end 120.916855 81.339836) (width 0.2) (layer "F.Cu") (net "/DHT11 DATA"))
 (segment (start 136.425 103.34) (end 100.38 103.34) (width 0.2) (layer "F.Cu") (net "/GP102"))
 (segment (start 100.38 103.34) (end 97.96 100.92) (width 0.2) (layer "F.Cu") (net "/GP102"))
 (segment (start 110.04 112.96) (end 113.5 109.5) (width 0.2) (layer "F.Cu") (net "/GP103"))
 (segment (start 110.396855 122.839735) (end 110.396855 121.679937) (width 0.2) (layer "F.Cu") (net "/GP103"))
 (segment (start 127 109.5) (end 128.5 108) (width 0.2) (layer "F.Cu") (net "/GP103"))
 (segment (start 113.5 109.5) (end 127 109.5) (width 0.2) (layer "F.Cu") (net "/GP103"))
 (segment (start 110.04 121.92) (end 110.04 112.96) (width 0.2) (layer "F.Cu") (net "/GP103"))
 (segment (start 128.5 108) (end 130.5 108) (width 0.2) (layer "F.Cu") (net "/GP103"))
 (segment (start 132.62 105.88) (end 136.425 105.88) (width 0.2) (layer "F.Cu") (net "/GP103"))
 (segment (start 130.5 108) (end 132.62 105.88) (width 0.2) (layer "F.Cu") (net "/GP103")))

